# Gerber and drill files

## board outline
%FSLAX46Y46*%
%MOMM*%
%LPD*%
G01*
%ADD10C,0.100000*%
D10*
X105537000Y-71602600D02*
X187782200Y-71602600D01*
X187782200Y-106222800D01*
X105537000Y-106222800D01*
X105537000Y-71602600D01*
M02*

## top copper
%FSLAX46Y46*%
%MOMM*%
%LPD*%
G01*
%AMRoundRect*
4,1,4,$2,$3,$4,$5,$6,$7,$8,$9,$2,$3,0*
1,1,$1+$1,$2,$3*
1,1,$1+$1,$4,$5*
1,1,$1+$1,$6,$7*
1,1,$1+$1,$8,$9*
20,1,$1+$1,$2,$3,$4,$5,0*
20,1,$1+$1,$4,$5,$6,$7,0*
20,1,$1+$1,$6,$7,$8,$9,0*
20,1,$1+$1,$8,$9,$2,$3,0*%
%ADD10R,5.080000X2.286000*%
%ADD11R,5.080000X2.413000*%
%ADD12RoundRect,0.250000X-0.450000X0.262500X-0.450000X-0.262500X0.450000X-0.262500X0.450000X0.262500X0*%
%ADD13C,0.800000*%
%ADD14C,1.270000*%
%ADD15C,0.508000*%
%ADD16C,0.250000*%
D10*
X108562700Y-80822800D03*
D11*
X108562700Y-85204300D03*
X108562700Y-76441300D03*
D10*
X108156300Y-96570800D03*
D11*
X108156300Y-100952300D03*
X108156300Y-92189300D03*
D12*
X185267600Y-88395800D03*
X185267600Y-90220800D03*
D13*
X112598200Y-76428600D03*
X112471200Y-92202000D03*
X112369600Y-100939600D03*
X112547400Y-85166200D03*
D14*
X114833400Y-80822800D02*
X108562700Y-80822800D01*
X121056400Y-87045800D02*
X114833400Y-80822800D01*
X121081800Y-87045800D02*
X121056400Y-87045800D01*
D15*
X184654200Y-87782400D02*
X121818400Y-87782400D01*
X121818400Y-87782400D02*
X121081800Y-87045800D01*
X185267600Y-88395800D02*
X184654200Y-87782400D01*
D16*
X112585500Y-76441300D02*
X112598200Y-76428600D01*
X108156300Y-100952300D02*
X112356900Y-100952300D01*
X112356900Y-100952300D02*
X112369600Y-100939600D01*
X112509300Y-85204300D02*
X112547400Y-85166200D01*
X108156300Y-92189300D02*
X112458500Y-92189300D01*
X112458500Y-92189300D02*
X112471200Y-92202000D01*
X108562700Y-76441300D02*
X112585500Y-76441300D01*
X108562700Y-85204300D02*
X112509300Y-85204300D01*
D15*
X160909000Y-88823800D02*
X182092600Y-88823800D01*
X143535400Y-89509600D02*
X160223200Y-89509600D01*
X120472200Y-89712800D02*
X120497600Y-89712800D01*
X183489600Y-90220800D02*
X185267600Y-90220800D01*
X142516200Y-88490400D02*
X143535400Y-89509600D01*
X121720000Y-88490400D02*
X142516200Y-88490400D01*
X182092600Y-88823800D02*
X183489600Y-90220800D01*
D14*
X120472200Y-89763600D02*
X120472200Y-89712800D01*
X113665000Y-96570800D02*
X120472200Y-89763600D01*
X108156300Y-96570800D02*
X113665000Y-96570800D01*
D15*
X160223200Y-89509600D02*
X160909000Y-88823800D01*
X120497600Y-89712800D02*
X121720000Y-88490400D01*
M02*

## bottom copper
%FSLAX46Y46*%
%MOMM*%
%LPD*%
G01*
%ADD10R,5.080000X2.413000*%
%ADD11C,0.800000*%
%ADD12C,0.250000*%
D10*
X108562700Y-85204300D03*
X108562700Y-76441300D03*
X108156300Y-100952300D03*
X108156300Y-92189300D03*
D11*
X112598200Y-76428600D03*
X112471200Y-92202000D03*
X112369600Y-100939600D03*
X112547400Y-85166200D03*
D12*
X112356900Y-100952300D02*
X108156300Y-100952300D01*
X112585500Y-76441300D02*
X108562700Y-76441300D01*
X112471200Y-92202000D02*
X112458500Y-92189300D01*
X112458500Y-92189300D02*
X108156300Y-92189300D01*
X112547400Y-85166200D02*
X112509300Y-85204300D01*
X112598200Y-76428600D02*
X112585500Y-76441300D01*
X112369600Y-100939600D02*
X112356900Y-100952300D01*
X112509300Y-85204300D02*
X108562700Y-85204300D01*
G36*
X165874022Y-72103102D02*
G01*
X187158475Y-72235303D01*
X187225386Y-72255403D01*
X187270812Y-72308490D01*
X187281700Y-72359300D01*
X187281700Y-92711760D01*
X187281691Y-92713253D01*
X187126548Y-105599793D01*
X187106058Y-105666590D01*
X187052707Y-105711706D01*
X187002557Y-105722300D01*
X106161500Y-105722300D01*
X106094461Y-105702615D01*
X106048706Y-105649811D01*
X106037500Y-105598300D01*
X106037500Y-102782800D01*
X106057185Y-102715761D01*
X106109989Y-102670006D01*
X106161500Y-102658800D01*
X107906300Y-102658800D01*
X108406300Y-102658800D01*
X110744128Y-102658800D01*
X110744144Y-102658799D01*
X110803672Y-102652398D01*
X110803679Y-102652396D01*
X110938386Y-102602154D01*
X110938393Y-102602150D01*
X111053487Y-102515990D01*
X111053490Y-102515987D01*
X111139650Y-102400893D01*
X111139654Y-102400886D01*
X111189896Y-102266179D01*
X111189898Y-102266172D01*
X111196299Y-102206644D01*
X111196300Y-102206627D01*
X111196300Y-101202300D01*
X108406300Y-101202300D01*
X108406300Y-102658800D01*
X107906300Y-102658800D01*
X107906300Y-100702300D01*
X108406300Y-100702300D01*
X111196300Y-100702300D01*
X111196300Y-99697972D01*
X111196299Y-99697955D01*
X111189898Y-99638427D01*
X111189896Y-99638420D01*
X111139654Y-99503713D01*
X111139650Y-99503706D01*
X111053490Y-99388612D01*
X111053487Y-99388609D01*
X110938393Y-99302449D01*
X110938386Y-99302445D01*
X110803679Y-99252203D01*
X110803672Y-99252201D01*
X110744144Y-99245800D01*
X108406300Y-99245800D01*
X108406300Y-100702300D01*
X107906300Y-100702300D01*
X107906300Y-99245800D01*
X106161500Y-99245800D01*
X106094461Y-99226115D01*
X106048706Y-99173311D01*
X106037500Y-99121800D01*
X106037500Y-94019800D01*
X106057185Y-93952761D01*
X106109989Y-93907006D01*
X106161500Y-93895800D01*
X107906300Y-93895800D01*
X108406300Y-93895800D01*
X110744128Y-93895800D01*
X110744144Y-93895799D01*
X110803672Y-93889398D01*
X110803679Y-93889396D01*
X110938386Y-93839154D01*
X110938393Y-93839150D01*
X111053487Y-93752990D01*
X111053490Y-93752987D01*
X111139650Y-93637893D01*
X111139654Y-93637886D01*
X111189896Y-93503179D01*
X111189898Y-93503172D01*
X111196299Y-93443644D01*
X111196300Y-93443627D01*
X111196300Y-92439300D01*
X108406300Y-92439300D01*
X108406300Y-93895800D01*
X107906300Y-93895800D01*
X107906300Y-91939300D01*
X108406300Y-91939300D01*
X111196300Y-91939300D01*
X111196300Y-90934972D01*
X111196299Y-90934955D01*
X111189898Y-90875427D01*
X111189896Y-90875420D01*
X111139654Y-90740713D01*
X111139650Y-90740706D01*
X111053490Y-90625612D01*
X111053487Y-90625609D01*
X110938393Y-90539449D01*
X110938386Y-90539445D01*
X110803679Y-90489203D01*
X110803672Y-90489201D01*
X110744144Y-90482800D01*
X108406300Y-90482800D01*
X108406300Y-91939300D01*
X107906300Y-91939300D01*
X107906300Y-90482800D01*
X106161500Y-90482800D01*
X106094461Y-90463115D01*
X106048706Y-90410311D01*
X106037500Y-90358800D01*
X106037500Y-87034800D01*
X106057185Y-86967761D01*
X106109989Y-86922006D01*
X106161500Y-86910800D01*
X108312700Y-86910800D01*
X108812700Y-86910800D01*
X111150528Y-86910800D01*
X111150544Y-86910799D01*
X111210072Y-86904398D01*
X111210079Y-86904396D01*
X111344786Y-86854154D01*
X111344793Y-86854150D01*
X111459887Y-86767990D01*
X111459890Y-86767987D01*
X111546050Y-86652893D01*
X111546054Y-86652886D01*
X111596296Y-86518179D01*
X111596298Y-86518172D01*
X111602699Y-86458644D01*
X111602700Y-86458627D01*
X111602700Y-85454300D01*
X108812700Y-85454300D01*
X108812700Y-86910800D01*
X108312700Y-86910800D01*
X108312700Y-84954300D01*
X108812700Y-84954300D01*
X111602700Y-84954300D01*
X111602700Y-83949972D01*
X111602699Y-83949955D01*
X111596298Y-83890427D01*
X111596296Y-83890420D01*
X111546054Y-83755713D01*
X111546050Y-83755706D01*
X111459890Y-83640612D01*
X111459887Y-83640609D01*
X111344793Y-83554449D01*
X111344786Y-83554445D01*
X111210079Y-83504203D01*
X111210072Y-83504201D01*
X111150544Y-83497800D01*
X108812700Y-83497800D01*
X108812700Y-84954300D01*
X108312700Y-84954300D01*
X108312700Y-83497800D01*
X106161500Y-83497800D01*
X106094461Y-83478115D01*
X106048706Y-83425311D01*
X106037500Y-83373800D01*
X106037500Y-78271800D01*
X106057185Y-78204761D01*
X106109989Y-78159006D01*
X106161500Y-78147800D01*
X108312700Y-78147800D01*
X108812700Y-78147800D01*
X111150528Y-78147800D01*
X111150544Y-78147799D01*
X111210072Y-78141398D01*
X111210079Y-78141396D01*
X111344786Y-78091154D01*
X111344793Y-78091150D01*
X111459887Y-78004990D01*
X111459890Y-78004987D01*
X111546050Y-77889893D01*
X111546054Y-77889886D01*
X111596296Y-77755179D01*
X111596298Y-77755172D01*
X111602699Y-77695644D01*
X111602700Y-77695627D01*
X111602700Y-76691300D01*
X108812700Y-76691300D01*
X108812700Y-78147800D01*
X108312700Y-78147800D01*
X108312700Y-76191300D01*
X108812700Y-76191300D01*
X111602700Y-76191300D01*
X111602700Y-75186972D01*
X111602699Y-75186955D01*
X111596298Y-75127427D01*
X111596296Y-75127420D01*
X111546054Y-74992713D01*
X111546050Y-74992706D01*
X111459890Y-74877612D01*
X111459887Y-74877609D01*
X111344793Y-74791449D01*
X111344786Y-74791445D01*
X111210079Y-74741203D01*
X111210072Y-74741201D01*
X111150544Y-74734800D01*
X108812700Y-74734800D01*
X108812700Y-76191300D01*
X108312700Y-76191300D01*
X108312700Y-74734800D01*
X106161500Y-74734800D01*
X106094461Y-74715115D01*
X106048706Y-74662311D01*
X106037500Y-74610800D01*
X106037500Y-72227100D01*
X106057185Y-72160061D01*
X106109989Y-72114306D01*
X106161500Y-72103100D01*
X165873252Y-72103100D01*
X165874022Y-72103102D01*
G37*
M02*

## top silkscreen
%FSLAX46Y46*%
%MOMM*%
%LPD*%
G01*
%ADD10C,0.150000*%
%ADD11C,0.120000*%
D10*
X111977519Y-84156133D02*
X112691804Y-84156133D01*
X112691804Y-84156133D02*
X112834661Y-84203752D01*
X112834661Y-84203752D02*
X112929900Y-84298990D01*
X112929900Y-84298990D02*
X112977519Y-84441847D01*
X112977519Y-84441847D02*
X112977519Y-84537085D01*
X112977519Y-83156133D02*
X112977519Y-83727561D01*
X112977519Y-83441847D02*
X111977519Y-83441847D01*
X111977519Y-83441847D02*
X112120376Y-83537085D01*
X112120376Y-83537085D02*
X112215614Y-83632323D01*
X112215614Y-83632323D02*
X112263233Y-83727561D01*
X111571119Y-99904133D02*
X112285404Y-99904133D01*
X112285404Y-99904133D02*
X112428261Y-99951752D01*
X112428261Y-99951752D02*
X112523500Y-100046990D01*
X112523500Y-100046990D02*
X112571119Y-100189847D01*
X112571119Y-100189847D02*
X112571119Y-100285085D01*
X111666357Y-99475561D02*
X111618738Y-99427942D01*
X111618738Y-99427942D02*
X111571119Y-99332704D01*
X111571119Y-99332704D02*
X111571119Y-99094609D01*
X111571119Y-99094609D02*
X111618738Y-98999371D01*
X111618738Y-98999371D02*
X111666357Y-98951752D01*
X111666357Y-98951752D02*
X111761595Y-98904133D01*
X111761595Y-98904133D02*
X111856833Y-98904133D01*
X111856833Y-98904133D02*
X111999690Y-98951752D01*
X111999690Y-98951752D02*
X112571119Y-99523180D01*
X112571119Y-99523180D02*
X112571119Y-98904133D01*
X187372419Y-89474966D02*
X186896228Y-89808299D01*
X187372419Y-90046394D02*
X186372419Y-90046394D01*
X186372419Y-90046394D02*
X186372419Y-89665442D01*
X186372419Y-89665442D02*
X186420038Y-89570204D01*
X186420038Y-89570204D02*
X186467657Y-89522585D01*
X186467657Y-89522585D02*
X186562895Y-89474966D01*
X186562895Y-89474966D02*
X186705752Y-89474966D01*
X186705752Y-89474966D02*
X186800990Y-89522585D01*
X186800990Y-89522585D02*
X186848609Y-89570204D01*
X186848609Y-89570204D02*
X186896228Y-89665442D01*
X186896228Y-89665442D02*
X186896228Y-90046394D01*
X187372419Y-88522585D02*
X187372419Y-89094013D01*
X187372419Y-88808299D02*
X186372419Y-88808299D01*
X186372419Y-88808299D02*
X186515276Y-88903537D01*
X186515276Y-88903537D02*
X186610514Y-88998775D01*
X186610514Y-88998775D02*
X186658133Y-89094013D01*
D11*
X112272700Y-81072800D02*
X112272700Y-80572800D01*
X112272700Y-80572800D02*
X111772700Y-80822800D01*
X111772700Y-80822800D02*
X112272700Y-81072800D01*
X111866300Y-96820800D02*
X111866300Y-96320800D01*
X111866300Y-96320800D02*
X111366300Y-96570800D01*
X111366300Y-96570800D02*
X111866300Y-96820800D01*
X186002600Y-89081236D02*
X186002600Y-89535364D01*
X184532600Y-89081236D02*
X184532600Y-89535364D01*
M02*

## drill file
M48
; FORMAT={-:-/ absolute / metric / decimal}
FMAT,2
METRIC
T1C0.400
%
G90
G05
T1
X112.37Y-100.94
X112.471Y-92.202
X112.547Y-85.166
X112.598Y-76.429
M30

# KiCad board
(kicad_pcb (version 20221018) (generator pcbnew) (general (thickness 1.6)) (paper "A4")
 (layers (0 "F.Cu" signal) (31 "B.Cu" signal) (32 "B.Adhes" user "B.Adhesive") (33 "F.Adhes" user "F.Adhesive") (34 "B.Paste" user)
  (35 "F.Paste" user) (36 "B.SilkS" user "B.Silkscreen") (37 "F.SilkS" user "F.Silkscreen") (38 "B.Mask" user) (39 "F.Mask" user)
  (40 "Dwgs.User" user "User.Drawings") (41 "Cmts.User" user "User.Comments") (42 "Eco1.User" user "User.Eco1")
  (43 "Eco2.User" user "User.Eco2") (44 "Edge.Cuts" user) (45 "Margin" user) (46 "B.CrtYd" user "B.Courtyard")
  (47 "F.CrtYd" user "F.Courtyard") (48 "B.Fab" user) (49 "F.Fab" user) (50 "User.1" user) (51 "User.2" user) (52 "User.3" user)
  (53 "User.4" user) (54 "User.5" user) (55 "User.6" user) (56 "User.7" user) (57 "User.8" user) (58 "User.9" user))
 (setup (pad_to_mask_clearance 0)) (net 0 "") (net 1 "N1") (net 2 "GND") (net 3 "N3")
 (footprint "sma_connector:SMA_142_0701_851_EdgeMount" (layer "F.Cu") (at 108.5627 80.8228 180)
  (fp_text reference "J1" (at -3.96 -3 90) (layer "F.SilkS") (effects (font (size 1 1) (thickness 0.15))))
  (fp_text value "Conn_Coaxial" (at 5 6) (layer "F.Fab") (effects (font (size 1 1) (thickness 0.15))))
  (fp_line (start -3.71 -0.25) (end -3.71 0.25) (stroke (width 0.12) (type solid)) (layer "F.SilkS"))
  (fp_line (start -3.71 0.25) (end -3.21 0) (stroke (width 0.12) (type solid)) (layer "F.SilkS"))
  (fp_line (start -3.21 0) (end -3.71 -0.25) (stroke (width 0.12) (type solid)) (layer "F.SilkS"))
  (pad "1" smd rect (at 0 0 270) (size 2.286 5.08) (layers "F.Cu" "F.Paste" "F.Mask") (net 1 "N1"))
  (pad "2" smd rect (at 0 -4.3815 270) (size 2.413 5.08) (layers "F.Cu" "F.Paste" "F.Mask") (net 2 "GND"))
  (pad "2" smd rect (at 0 -4.3815 270) (size 2.413 5.08) (layers "B.Cu" "B.Paste" "B.Mask") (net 2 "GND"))
  (pad "2" smd rect (at 0 4.3815 270) (size 2.413 5.08) (layers "F.Cu" "F.Paste" "F.Mask") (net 2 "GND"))
  (pad "2" smd rect (at 0 4.3815 270) (size 2.413 5.08) (layers "B.Cu" "B.Paste" "B.Mask") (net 2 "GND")))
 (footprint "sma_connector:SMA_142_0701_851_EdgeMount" (layer "F.Cu") (at 108.1563 96.5708 180)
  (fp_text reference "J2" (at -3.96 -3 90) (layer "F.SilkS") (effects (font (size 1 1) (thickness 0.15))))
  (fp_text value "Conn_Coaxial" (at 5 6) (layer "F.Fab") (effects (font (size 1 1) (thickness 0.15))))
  (fp_line (start -3.71 -0.25) (end -3.71 0.25) (stroke (width 0.12) (type solid)) (layer "F.SilkS"))
  (fp_line (start -3.71 0.25) (end -3.21 0) (stroke (width 0.12) (type solid)) (layer "F.SilkS"))
  (fp_line (start -3.21 0) (end -3.71 -0.25) (stroke (width 0.12) (type solid)) (layer "F.SilkS"))
  (pad "1" smd rect (at 0 0 270) (size 2.286 5.08) (layers "F.Cu" "F.Paste" "F.Mask") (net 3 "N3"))
  (pad "2" smd rect (at 0 -4.3815 270) (size 2.413 5.08) (layers "F.Cu" "F.Paste" "F.Mask") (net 2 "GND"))
  (pad "2" smd rect (at 0 -4.3815 270) (size 2.413 5.08) (layers "B.Cu" "B.Paste" "B.Mask") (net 2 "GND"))
  (pad "2" smd rect (at 0 4.3815 270) (size 2.413 5.08) (layers "F.Cu" "F.Paste" "F.Mask") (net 2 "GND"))
  (pad "2" smd rect (at 0 4.3815 270) (size 2.413 5.08) (layers "B.Cu" "B.Paste" "B.Mask") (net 2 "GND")))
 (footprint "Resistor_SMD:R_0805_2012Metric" (layer "F.Cu") (at 185.2676 89.3083 -90)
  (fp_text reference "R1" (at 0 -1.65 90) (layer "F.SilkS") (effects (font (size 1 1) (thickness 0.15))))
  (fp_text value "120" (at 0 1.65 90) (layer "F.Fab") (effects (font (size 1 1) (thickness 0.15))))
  (fp_line (start -0.227064 -0.735) (end 0.227064 -0.735) (stroke (width 0.12) (type solid)) (layer "F.SilkS"))
  (fp_line (start -0.227064 0.735) (end 0.227064 0.735) (stroke (width 0.12) (type solid)) (layer "F.SilkS"))
  (pad "1" smd roundrect (at -0.9125 0 270) (size 1.025 1.4) (layers "F.Cu" "F.Paste" "F.Mask") (roundrect_rratio 0.243902) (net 1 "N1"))
  (pad "2" smd roundrect (at 0.9125 0 270) (size 1.025 1.4) (layers "F.Cu" "F.Paste" "F.Mask") (roundrect_rratio 0.243902) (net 3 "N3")))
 (gr_rect (start 105.537 71.6026) (end 187.7822 106.2228) (stroke (width 0.1) (type default)) (fill none) (layer "Edge.Cuts"))
 (segment (start 114.8334 80.8228) (end 108.5627 80.8228) (width 1.27) (layer "F.Cu") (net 1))
 (segment (start 121.0564 87.0458) (end 114.8334 80.8228) (width 1.27) (layer "F.Cu") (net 1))
 (segment (start 121.0818 87.0458) (end 121.0564 87.0458) (width 1.27) (layer "F.Cu") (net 1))
 (segment (start 184.6542 87.7824) (end 121.8184 87.7824) (width 0.508) (layer "F.Cu") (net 1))
 (segment (start 121.8184 87.7824) (end 121.0818 87.0458) (width 0.508) (layer "F.Cu") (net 1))
 (segment (start 185.2676 88.3958) (end 184.6542 87.7824) (width 0.508) (layer "F.Cu") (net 1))
 (segment (start 112.5855 76.4413) (end 112.5982 76.4286) (width 0.25) (layer "F.Cu") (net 2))
 (segment (start 108.1563 100.9523) (end 112.3569 100.9523) (width 0.25) (layer "F.Cu") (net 2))
 (segment (start 112.3569 100.9523) (end 112.3696 100.9396) (width 0.25) (layer "F.Cu") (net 2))
 (segment (start 112.5093 85.2043) (end 112.5474 85.1662) (width 0.25) (layer "F.Cu") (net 2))
 (segment (start 108.1563 92.1893) (end 112.4585 92.1893) (width 0.25) (layer "F.Cu") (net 2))
 (segment (start 112.4585 92.1893) (end 112.4712 92.202) (width 0.25) (layer "F.Cu") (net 2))
 (segment (start 108.5627 76.4413) (end 112.5855 76.4413) (width 0.25) (layer "F.Cu") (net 2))
 (segment (start 108.5627 85.2043) (end 112.5093 85.2043) (width 0.25) (layer "F.Cu") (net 2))
 (via (at 112.5982 76.4286) (size 0.8) (drill 0.4) (layers "F.Cu" "B.Cu") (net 2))
 (via (at 112.4712 92.202) (size 0.8) (drill 0.4) (layers "F.Cu" "B.Cu") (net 2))
 (via (at 112.3696 100.9396) (size 0.8) (drill 0.4) (layers "F.Cu" "B.Cu") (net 2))
 (via (at 112.5474 85.1662) (size 0.8) (drill 0.4) (layers "F.Cu" "B.Cu") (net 2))
 (segment (start 112.3569 100.9523) (end 108.1563 100.9523) (width 0.25) (layer "B.Cu") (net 2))
 (segment (start 112.5855 76.4413) (end 108.5627 76.4413) (width 0.25) (layer "B.Cu") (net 2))
 (segment (start 112.4712 92.202) (end 112.4585 92.1893) (width 0.25) (layer "B.Cu") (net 2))
 (segment (start 112.4585 92.1893) (end 108.1563 92.1893) (width 0.25) (layer "B.Cu") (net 2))
 (segment (start 112.5474 85.1662) (end 112.5093 85.2043) (width 0.25) (layer "B.Cu") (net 2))
 (segment (start 112.5982 76.4286) (end 112.5855 76.4413) (width 0.25) (layer "B.Cu") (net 2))
 (segment (start 112.3696 100.9396) (end 112.3569 100.9523) (width 0.25) (layer "B.Cu") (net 2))
 (segment (start 112.5093 85.2043) (end 108.5627 85.2043) (width 0.25) (layer "B.Cu") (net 2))
 (segment (start 160.909 88.8238) (end 182.0926 88.8238) (width 0.508) (layer "F.Cu") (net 3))
 (segment (start 143.5354 89.5096) (end 160.2232 89.5096) (width 0.508) (layer "F.Cu") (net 3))
 (segment (start 120.4722 89.7128) (end 120.4976 89.7128) (width 0.508) (layer "F.Cu") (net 3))
 (segment (start 183.4896 90.2208) (end 185.2676 90.2208) (width 0.508) (layer "F.Cu") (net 3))
 (segment (start 142.5162 88.4904) (end 143.5354 89.5096) (width 0.508) (layer "F.Cu") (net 3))
 (segment (start 121.72 88.4904) (end 142.5162 88.4904) (width 0.508) (layer "F.Cu") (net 3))
 (segment (start 182.0926 88.8238) (end 183.4896 90.2208) (width 0.508) (layer "F.Cu") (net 3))
 (segment (start 120.4722 89.7636) (end 120.4722 89.7128) (width 1.27) (layer "F.Cu") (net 3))
 (segment (start 113.665 96.5708) (end 120.4722 89.7636) (width 1.27) (layer "F.Cu") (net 3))
 (segment (start 108.1563 96.5708) (end 113.665 96.5708) (width 1.27) (layer "F.Cu") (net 3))
 (segment (start 160.2232 89.5096) (end 160.909 88.8238) (width 0.508) (layer "F.Cu") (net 3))
 (segment (start 120.4976 89.7128) (end 121.72 88.4904) (width 0.508) (layer "F.Cu") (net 3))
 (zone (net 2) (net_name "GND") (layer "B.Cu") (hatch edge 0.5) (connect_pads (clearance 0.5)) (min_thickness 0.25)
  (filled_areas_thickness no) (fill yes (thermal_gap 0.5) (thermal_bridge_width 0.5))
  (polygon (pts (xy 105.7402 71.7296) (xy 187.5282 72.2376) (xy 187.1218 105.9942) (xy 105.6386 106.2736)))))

